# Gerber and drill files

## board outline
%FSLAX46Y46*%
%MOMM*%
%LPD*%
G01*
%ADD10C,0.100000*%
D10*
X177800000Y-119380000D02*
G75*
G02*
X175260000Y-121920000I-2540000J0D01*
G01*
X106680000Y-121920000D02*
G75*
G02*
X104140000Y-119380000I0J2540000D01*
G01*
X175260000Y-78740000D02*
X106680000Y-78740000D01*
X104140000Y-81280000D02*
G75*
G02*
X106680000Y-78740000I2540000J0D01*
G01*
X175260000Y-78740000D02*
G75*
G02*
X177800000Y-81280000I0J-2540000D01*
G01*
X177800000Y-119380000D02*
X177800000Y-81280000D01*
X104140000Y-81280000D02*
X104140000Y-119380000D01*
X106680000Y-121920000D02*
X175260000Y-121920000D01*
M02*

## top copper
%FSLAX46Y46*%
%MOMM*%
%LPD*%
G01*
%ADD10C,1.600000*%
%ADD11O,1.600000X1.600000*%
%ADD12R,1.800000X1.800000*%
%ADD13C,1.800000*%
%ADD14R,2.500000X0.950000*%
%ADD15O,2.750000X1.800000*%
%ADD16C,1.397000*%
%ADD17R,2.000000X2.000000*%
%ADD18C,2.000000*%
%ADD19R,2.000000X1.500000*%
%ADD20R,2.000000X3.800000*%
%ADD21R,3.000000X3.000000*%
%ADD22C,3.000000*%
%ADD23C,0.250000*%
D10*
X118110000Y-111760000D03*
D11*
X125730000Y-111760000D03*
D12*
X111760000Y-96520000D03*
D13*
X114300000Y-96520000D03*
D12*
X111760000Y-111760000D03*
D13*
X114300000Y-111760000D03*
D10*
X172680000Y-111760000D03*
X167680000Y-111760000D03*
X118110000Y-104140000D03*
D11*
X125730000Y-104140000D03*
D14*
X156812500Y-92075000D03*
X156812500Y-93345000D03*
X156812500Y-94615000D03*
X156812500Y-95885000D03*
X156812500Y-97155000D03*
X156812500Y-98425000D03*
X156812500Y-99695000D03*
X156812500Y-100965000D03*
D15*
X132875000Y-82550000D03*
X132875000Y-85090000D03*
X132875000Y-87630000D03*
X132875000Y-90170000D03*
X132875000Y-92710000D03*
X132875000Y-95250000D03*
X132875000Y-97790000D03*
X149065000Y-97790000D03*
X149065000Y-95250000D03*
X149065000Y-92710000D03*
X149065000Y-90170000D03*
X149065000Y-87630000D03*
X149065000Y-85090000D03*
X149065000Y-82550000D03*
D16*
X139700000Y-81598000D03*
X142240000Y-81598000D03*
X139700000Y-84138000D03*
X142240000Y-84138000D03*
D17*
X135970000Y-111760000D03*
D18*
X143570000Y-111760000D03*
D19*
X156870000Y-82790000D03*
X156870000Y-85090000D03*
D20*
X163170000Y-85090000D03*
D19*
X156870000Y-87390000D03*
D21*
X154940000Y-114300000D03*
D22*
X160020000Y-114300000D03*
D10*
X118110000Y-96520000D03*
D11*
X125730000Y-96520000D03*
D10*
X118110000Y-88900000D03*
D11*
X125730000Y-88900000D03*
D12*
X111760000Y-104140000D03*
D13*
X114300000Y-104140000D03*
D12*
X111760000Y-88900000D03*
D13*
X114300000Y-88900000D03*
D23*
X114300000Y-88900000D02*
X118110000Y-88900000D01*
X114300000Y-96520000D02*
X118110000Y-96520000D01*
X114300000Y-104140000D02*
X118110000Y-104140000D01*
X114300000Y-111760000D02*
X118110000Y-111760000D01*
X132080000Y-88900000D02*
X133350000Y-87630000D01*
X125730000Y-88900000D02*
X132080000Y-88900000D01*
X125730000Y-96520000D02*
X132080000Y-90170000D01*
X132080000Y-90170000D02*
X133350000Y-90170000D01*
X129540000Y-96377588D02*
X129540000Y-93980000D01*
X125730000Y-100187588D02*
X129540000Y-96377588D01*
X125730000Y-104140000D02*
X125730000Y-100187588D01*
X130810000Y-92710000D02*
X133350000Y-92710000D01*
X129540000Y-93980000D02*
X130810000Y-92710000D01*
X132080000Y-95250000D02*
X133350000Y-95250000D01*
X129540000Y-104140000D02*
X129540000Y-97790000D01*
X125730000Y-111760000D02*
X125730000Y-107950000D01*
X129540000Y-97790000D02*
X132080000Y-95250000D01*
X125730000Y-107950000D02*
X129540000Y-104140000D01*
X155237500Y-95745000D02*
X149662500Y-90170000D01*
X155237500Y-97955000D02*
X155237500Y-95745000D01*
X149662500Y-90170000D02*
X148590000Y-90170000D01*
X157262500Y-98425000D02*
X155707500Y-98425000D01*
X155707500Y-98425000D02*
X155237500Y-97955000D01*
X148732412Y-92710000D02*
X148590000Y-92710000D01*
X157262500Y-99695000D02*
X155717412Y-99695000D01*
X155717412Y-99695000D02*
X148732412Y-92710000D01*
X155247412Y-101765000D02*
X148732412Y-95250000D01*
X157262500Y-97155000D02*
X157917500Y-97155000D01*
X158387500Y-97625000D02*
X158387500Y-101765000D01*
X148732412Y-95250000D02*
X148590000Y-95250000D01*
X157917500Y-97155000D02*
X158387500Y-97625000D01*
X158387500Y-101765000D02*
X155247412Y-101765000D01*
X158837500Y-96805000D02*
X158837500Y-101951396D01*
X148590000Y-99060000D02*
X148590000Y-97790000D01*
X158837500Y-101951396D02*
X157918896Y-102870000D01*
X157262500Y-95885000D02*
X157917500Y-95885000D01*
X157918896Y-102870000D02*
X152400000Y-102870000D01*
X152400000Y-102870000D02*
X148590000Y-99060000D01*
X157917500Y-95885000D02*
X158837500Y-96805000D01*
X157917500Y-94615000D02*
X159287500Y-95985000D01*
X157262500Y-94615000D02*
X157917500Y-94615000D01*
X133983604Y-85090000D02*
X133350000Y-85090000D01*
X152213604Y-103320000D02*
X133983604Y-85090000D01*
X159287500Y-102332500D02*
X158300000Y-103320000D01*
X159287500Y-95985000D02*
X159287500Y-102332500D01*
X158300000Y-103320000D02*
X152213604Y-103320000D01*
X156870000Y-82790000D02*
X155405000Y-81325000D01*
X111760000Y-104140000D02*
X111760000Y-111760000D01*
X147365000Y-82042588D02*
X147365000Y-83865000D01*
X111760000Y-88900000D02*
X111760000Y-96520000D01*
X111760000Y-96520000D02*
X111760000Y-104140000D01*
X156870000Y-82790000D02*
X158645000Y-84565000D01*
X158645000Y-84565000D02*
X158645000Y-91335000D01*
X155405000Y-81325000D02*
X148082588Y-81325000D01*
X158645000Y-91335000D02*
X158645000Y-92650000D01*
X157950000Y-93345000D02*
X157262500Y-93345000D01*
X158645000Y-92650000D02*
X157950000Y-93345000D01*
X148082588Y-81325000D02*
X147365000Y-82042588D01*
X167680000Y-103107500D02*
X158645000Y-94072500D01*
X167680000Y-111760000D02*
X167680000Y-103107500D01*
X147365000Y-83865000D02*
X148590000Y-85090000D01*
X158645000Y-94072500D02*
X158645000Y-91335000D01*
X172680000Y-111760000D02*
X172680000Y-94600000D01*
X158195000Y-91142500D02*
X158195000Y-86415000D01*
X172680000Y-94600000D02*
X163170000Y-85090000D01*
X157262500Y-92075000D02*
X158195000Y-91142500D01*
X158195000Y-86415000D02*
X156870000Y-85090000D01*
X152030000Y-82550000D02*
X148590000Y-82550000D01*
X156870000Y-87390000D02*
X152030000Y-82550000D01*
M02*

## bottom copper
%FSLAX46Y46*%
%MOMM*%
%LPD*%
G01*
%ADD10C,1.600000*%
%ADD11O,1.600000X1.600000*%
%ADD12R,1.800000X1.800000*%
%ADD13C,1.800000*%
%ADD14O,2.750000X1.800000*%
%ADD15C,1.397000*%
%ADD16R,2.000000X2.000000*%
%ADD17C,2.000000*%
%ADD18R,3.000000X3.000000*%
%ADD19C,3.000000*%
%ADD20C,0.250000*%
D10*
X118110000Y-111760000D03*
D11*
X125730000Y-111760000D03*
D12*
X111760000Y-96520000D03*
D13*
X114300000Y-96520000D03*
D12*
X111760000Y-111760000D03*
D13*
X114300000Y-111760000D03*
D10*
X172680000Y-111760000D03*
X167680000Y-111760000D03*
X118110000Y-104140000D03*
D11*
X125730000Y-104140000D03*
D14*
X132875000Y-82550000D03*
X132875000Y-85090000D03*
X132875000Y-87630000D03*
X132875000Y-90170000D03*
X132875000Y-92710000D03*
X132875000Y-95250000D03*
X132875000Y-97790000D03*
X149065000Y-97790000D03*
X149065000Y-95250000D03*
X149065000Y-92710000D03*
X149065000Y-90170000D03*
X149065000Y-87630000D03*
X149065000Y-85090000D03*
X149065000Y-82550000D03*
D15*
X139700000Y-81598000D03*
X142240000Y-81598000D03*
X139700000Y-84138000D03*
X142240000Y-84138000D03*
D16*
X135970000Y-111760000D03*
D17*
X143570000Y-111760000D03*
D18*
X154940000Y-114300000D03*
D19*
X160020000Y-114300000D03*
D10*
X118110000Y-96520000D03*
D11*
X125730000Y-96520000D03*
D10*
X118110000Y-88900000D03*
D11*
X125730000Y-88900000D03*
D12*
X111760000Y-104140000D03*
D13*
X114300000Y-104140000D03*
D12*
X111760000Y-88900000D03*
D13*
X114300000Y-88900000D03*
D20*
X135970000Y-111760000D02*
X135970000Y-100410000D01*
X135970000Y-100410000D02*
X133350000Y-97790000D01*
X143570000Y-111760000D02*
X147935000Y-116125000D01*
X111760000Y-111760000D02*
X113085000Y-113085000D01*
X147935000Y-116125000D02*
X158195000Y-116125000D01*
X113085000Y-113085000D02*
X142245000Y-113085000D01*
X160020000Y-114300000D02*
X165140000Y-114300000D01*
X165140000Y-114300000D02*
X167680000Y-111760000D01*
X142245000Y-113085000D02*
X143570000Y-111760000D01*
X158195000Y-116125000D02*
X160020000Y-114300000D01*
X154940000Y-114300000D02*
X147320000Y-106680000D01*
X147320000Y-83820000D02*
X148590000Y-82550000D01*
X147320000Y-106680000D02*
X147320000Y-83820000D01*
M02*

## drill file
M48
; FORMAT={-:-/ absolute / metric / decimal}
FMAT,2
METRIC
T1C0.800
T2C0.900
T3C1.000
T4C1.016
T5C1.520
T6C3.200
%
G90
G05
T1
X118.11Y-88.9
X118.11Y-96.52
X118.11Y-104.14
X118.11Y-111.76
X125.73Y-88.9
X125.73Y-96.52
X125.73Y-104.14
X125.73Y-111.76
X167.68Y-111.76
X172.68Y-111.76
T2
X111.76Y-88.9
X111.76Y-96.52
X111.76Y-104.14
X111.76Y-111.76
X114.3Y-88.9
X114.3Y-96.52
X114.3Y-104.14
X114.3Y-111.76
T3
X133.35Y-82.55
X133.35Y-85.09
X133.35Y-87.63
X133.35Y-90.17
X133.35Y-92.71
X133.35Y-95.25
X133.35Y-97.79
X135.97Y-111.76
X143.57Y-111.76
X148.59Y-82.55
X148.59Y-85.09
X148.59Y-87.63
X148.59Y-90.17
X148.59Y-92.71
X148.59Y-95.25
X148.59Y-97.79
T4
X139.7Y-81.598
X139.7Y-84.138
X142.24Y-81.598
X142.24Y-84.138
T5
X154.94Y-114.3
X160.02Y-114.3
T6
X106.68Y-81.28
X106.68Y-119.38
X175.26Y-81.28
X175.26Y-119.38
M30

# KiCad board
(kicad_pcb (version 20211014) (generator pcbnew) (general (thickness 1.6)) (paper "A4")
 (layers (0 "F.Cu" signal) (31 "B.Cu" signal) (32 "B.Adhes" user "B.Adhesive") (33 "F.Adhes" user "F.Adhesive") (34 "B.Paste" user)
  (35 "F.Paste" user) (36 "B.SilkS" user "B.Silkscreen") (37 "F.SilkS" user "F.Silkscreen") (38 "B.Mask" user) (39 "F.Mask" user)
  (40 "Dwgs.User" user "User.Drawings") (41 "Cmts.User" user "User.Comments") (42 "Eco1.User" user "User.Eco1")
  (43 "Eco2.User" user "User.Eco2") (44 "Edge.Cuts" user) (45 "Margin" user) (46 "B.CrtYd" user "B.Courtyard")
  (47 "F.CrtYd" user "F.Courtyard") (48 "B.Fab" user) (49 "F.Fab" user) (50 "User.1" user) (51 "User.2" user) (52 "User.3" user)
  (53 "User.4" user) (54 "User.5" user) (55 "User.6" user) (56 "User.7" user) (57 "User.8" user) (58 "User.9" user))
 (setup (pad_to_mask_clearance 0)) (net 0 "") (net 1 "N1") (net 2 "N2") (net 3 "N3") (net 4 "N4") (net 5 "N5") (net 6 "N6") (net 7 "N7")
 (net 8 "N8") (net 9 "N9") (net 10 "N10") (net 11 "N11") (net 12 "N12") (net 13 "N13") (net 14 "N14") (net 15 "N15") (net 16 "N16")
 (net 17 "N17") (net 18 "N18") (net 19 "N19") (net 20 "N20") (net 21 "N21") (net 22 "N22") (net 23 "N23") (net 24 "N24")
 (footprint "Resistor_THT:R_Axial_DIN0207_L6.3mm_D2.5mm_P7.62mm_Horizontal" (layer "F.Cu") (at 118.11 111.76)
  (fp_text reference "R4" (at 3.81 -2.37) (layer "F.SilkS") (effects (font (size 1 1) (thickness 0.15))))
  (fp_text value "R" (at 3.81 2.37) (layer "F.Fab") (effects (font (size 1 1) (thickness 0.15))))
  (pad "1" thru_hole circle (at 0 0) (size 1.6 1.6) (drill 0.8) (layers *.Cu *.Mask) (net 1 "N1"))
  (pad "2" thru_hole oval (at 7.62 0) (size 1.6 1.6) (drill 0.8) (layers *.Cu *.Mask) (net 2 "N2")))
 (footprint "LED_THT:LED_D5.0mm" (layer "F.Cu") (at 111.76 96.52)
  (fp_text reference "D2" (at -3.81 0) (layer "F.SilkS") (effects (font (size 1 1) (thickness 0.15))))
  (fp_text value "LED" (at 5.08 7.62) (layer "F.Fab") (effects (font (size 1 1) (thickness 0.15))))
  (pad "1" thru_hole rect (at 0 0) (size 1.8 1.8) (drill 0.9) (layers *.Cu *.Mask) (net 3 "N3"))
  (pad "2" thru_hole circle (at 2.54 0) (size 1.8 1.8) (drill 0.9) (layers *.Cu *.Mask) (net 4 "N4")))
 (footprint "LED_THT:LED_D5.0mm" (layer "F.Cu") (at 111.76 111.76)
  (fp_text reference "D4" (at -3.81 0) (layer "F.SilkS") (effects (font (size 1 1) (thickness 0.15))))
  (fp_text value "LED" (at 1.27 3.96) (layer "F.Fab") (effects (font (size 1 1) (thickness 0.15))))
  (pad "1" thru_hole rect (at 0 0) (size 1.8 1.8) (drill 0.9) (layers *.Cu *.Mask) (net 3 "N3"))
  (pad "2" thru_hole circle (at 2.54 0) (size 1.8 1.8) (drill 0.9) (layers *.Cu *.Mask) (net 1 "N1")))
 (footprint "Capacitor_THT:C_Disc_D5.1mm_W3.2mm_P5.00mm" (layer "F.Cu") (at 172.68 111.76 180)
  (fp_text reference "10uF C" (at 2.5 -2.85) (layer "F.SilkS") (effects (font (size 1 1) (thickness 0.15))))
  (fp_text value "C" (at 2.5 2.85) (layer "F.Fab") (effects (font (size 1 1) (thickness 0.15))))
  (pad "1" thru_hole circle (at 0 0 180) (size 1.6 1.6) (drill 0.8) (layers *.Cu *.Mask) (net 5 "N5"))
  (pad "2" thru_hole circle (at 5 0 180) (size 1.6 1.6) (drill 0.8) (layers *.Cu *.Mask) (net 3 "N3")))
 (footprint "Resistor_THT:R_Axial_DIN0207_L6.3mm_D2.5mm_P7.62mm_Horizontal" (layer "F.Cu") (at 118.11 104.14)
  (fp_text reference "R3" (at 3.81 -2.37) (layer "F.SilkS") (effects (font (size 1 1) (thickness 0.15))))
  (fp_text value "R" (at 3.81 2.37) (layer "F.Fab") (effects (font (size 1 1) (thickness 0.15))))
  (pad "1" thru_hole circle (at 0 0) (size 1.6 1.6) (drill 0.8) (layers *.Cu *.Mask) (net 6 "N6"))
  (pad "2" thru_hole oval (at 7.62 0) (size 1.6 1.6) (drill 0.8) (layers *.Cu *.Mask) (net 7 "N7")))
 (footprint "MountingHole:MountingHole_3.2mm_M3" (layer "F.Cu") (at 106.68 119.38)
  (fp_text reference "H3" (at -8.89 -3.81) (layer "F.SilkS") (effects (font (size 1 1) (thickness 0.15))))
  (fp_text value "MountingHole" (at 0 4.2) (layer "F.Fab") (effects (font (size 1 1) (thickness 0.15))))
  (pad "" np_thru_hole circle (at 0 0) (size 3.2 3.2) (drill 3.2) (layers *.Cu *.Mask)))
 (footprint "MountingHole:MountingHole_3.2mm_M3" (layer "F.Cu") (at 106.68 81.28)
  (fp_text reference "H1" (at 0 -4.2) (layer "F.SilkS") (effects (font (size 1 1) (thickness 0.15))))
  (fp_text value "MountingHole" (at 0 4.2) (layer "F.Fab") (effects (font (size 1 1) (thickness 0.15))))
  (pad "" np_thru_hole circle (at 0 0) (size 3.2 3.2) (drill 3.2) (layers *.Cu *.Mask)))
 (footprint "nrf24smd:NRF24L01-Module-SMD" (layer "F.Cu") (at 157.5625 96.52 180)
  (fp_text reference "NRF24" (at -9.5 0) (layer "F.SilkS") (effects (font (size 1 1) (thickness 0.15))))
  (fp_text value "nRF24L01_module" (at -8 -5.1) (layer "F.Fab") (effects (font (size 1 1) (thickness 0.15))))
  (pad "1" smd rect locked (at 0.3 4.445 180) (size 2.5 0.95) (drill (offset 0.45 0)) (layers "F.Cu" "F.Paste" "F.Mask") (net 5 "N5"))
  (pad "2" smd rect locked (at 0.3 3.175 180) (size 2.5 0.95) (drill (offset 0.45 0)) (layers "F.Cu" "F.Paste" "F.Mask") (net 3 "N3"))
  (pad "3" smd rect locked (at 0.3 1.905 180) (size 2.5 0.95) (drill (offset 0.45 0)) (layers "F.Cu" "F.Paste" "F.Mask") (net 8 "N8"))
  (pad "4" smd rect locked (at 0.3 0.635 180) (size 2.5 0.95) (drill (offset 0.45 0)) (layers "F.Cu" "F.Paste" "F.Mask") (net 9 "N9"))
  (pad "5" smd rect locked (at 0.3 -0.635 180) (size 2.5 0.95) (drill (offset 0.45 0)) (layers "F.Cu" "F.Paste" "F.Mask") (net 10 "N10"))
  (pad "6" smd rect locked (at 0.3 -1.905 180) (size 2.5 0.95) (drill (offset 0.45 0)) (layers "F.Cu" "F.Paste" "F.Mask") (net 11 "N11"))
  (pad "7" smd rect locked (at 0.3 -3.175 180) (size 2.5 0.95) (drill (offset 0.45 0)) (layers "F.Cu" "F.Paste" "F.Mask") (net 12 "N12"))
  (pad "8" smd rect locked (at 0.3 -4.445 180) (size 2.5 0.95) (drill (offset 0.45 0)) (layers "F.Cu" "F.Paste" "F.Mask") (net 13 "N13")))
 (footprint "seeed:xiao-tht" (layer "F.Cu") (at 140.97 90.17)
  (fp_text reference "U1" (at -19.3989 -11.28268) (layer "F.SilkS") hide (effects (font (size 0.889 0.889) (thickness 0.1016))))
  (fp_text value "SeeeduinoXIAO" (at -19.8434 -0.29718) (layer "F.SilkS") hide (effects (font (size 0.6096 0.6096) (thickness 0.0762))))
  (pad "1" thru_hole oval (at -7.62 -7.62) (size 2.75 1.8) (drill 1 (offset -0.475 0)) (layers *.Cu *.Mask) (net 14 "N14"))
  (pad "2" thru_hole oval (at -7.62 -5.08) (size 2.75 1.8) (drill 1 (offset -0.475 0)) (layers *.Cu *.Mask) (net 8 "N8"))
  (pad "3" thru_hole oval (at -7.62 -2.54) (size 2.75 1.8) (drill 1 (offset -0.475 0)) (layers *.Cu *.Mask) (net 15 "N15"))
  (pad "4" thru_hole oval (at -7.62 0) (size 2.75 1.8) (drill 1 (offset -0.475 0)) (layers *.Cu *.Mask) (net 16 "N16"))
  (pad "5" thru_hole oval (at -7.62 2.54) (size 2.75 1.8) (drill 1 (offset -0.475 0)) (layers *.Cu *.Mask) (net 7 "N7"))
  (pad "6" thru_hole oval (at -7.62 5.08) (size 2.75 1.8) (drill 1 (offset -0.475 0)) (layers *.Cu *.Mask) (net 2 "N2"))
  (pad "7" thru_hole oval (at -7.62 7.62) (size 2.75 1.8) (drill 1 (offset -0.475 0)) (layers *.Cu *.Mask) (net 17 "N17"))
  (pad "8" thru_hole oval (at 7.62 7.62 180) (size 2.75 1.8) (drill 1 (offset -0.475 0)) (layers *.Cu *.Mask) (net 9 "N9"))
  (pad "9" thru_hole oval (at 7.62 5.08 180) (size 2.75 1.8) (drill 1 (offset -0.475 0)) (layers *.Cu *.Mask) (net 10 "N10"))
  (pad "10" thru_hole oval (at 7.62 2.54 180) (size 2.75 1.8) (drill 1 (offset -0.475 0)) (layers *.Cu *.Mask) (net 12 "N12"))
  (pad "11" thru_hole oval (at 7.62 0 180) (size 2.75 1.8) (drill 1 (offset -0.475 0)) (layers *.Cu *.Mask) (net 11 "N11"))
  (pad "12" thru_hole oval (at 7.62 -2.54 180) (size 2.75 1.8) (drill 1 (offset -0.475 0)) (layers *.Cu *.Mask) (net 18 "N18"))
  (pad "13" thru_hole oval (at 7.62 -5.08 180) (size 2.75 1.8) (drill 1 (offset -0.475 0)) (layers *.Cu *.Mask) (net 3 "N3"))
  (pad "14" thru_hole oval (at 7.62 -7.62 180) (size 2.75 1.8) (drill 1 (offset -0.475 0)) (layers *.Cu *.Mask) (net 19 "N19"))
  (pad "15" thru_hole circle (at -1.27 -8.572 90) (size 1.397 1.397) (drill 1.016) (layers *.Cu *.Mask) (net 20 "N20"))
  (pad "16" thru_hole circle (at 1.27 -8.572 90) (size 1.397 1.397) (drill 1.016) (layers *.Cu *.Mask) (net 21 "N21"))
  (pad "17" thru_hole circle (at -1.27 -6.032 90) (size 1.397 1.397) (drill 1.016) (layers *.Cu *.Mask) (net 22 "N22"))
  (pad "18" thru_hole circle (at 1.27 -6.032 90) (size 1.397 1.397) (drill 1.016) (layers *.Cu *.Mask) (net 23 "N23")))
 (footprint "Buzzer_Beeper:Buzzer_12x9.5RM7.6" (layer "F.Cu") (at 135.97 111.76)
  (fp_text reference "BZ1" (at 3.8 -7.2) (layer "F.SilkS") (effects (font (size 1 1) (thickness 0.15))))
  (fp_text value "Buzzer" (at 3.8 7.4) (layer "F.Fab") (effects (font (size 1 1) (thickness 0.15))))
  (pad "1" thru_hole rect (at 0 0) (size 2 2) (drill 1) (layers *.Cu *.Mask) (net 17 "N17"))
  (pad "2" thru_hole circle (at 7.6 0) (size 2 2) (drill 1) (layers *.Cu *.Mask) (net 3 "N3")))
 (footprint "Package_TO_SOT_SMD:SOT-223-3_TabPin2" (layer "F.Cu") (at 160.02 85.09)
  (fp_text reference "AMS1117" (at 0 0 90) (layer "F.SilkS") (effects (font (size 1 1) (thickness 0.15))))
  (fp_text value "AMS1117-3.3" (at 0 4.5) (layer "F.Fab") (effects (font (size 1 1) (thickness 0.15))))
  (pad "1" smd rect (at -3.15 -2.3) (size 2 1.5) (layers "F.Cu" "F.Paste" "F.Mask") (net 3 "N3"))
  (pad "2" smd rect (at -3.15 0) (size 2 1.5) (layers "F.Cu" "F.Paste" "F.Mask") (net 5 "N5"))
  (pad "2" smd rect (at 3.15 0) (size 2 3.8) (layers "F.Cu" "F.Paste" "F.Mask") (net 5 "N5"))
  (pad "3" smd rect (at -3.15 2.3) (size 2 1.5) (layers "F.Cu" "F.Paste" "F.Mask") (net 19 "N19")))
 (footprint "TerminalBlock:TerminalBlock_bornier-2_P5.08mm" (layer "F.Cu") (at 154.94 114.3)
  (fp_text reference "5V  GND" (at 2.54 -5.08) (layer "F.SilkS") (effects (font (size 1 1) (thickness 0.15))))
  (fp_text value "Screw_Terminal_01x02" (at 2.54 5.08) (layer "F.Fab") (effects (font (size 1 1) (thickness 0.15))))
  (pad "1" thru_hole rect (at 0 0) (size 3 3) (drill 1.52) (layers *.Cu *.Mask) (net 19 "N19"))
  (pad "2" thru_hole circle (at 5.08 0) (size 3 3) (drill 1.52) (layers *.Cu *.Mask) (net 3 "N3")))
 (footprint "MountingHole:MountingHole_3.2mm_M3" (layer "F.Cu") (at 175.26 81.28)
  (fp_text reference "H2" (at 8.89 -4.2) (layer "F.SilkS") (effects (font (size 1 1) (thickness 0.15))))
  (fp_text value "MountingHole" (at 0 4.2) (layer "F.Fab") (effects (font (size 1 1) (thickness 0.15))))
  (pad "" np_thru_hole circle (at 0 0) (size 3.2 3.2) (drill 3.2) (layers *.Cu *.Mask)))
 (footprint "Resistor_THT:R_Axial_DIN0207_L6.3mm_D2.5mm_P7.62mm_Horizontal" (layer "F.Cu") (at 118.11 96.52)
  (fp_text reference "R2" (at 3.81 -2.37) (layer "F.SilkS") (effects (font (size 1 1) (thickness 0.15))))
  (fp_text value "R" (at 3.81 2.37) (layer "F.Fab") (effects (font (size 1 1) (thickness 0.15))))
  (pad "1" thru_hole circle (at 0 0) (size 1.6 1.6) (drill 0.8) (layers *.Cu *.Mask) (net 4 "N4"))
  (pad "2" thru_hole oval (at 7.62 0) (size 1.6 1.6) (drill 0.8) (layers *.Cu *.Mask) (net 16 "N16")))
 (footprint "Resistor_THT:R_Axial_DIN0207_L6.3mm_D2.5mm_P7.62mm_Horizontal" (layer "F.Cu") (at 118.11 88.9)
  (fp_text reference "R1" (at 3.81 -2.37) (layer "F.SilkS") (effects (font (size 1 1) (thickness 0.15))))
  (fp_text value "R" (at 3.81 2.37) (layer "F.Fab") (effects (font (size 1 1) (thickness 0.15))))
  (pad "1" thru_hole circle (at 0 0) (size 1.6 1.6) (drill 0.8) (layers *.Cu *.Mask) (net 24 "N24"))
  (pad "2" thru_hole oval (at 7.62 0) (size 1.6 1.6) (drill 0.8) (layers *.Cu *.Mask) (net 15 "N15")))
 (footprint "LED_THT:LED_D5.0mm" (layer "F.Cu") (at 111.76 104.14)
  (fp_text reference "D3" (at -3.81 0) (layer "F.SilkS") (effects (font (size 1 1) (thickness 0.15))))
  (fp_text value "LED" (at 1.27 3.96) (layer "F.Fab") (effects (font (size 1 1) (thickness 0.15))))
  (pad "1" thru_hole rect (at 0 0) (size 1.8 1.8) (drill 0.9) (layers *.Cu *.Mask) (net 3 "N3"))
  (pad "2" thru_hole circle (at 2.54 0) (size 1.8 1.8) (drill 0.9) (layers *.Cu *.Mask) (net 6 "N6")))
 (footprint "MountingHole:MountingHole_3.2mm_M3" (layer "F.Cu") (at 175.26 119.38)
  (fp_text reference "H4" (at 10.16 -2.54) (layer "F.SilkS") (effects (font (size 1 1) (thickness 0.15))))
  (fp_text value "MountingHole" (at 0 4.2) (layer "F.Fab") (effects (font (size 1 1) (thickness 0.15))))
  (pad "" np_thru_hole circle (at 0 0) (size 3.2 3.2) (drill 3.2) (layers *.Cu *.Mask)))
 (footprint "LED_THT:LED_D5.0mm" (layer "F.Cu") (at 111.76 88.9)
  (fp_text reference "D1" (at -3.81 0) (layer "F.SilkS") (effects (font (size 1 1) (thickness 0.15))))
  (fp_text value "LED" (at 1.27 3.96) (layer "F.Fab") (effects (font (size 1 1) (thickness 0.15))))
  (pad "1" thru_hole rect (at 0 0) (size 1.8 1.8) (drill 0.9) (layers *.Cu *.Mask) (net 3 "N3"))
  (pad "2" thru_hole circle (at 2.54 0) (size 1.8 1.8) (drill 0.9) (layers *.Cu *.Mask) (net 24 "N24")))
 (gr_arc (start 177.8 119.38) (mid 177.056051 121.176051) (end 175.26 121.92) (layer "Edge.Cuts") (width 0.1))
 (gr_arc (start 106.68 121.92) (mid 104.883949 121.176051) (end 104.14 119.38) (layer "Edge.Cuts") (width 0.1))
 (gr_line (start 175.26 78.74) (end 106.68 78.74) (layer "Edge.Cuts") (width 0.1))
 (gr_arc (start 104.14 81.28) (mid 104.883949 79.483949) (end 106.68 78.74) (layer "Edge.Cuts") (width 0.1))
 (gr_arc (start 175.26 78.74) (mid 177.056051 79.483949) (end 177.8 81.28) (layer "Edge.Cuts") (width 0.1))
 (gr_line (start 177.8 119.38) (end 177.8 81.28) (layer "Edge.Cuts") (width 0.1))
 (gr_line (start 104.14 81.28) (end 104.14 119.38) (layer "Edge.Cuts") (width 0.1))
 (gr_line (start 106.68 121.92) (end 175.26 121.92) (layer "Edge.Cuts") (width 0.1))
 (segment (start 114.3 88.9) (end 118.11 88.9) (width 0.25) (layer "F.Cu") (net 24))
 (segment (start 114.3 96.52) (end 118.11 96.52) (width 0.25) (layer "F.Cu") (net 4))
 (segment (start 114.3 104.14) (end 118.11 104.14) (width 0.25) (layer "F.Cu") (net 6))
 (segment (start 114.3 111.76) (end 118.11 111.76) (width 0.25) (layer "F.Cu") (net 1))
 (segment (start 132.08 88.9) (end 133.35 87.63) (width 0.25) (layer "F.Cu") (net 15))
 (segment (start 125.73 88.9) (end 132.08 88.9) (width 0.25) (layer "F.Cu") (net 15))
 (segment (start 125.73 96.52) (end 132.08 90.17) (width 0.25) (layer "F.Cu") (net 16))
 (segment (start 132.08 90.17) (end 133.35 90.17) (width 0.25) (layer "F.Cu") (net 16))
 (segment (start 129.54 96.377588) (end 129.54 93.98) (width 0.25) (layer "F.Cu") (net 7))
 (segment (start 125.73 100.187588) (end 129.54 96.377588) (width 0.25) (layer "F.Cu") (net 7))
 (segment (start 125.73 104.14) (end 125.73 100.187588) (width 0.25) (layer "F.Cu") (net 7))
 (segment (start 130.81 92.71) (end 133.35 92.71) (width 0.25) (layer "F.Cu") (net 7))
 (segment (start 129.54 93.98) (end 130.81 92.71) (width 0.25) (layer "F.Cu") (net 7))
 (segment (start 132.08 95.25) (end 133.35 95.25) (width 0.25) (layer "F.Cu") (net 2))
 (segment (start 129.54 104.14) (end 129.54 97.79) (width 0.25) (layer "F.Cu") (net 2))
 (segment (start 125.73 111.76) (end 125.73 107.95) (width 0.25) (layer "F.Cu") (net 2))
 (segment (start 129.54 97.79) (end 132.08 95.25) (width 0.25) (layer "F.Cu") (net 2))
 (segment (start 125.73 107.95) (end 129.54 104.14) (width 0.25) (layer "F.Cu") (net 2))
 (segment (start 155.2375 95.745) (end 149.6625 90.17) (width 0.25) (layer "F.Cu") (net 11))
 (segment (start 155.2375 97.955) (end 155.2375 95.745) (width 0.25) (layer "F.Cu") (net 11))
 (segment (start 149.6625 90.17) (end 148.59 90.17) (width 0.25) (layer "F.Cu") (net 11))
 (segment (start 157.2625 98.425) (end 155.7075 98.425) (width 0.25) (layer "F.Cu") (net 11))
 (segment (start 155.7075 98.425) (end 155.2375 97.955) (width 0.25) (layer "F.Cu") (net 11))
 (segment (start 148.732412 92.71) (end 148.59 92.71) (width 0.25) (layer "F.Cu") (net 12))
 (segment (start 157.2625 99.695) (end 155.717412 99.695) (width 0.25) (layer "F.Cu") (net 12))
 (segment (start 155.717412 99.695) (end 148.732412 92.71) (width 0.25) (layer "F.Cu") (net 12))
 (segment (start 155.247412 101.765) (end 148.732412 95.25) (width 0.25) (layer "F.Cu") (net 10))
 (segment (start 157.2625 97.155) (end 157.9175 97.155) (width 0.25) (layer "F.Cu") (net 10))
 (segment (start 158.3875 97.625) (end 158.3875 101.765) (width 0.25) (layer "F.Cu") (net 10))
 (segment (start 148.732412 95.25) (end 148.59 95.25) (width 0.25) (layer "F.Cu") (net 10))
 (segment (start 157.9175 97.155) (end 158.3875 97.625) (width 0.25) (layer "F.Cu") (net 10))
 (segment (start 158.3875 101.765) (end 155.247412 101.765) (width 0.25) (layer "F.Cu") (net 10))
 (segment (start 158.8375 96.805) (end 158.8375 101.951396) (width 0.25) (layer "F.Cu") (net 9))
 (segment (start 148.59 99.06) (end 148.59 97.79) (width 0.25) (layer "F.Cu") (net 9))
 (segment (start 158.8375 101.951396) (end 157.918896 102.87) (width 0.25) (layer "F.Cu") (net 9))
 (segment (start 157.2625 95.885) (end 157.9175 95.885) (width 0.25) (layer "F.Cu") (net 9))
 (segment (start 157.918896 102.87) (end 152.4 102.87) (width 0.25) (layer "F.Cu") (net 9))
 (segment (start 152.4 102.87) (end 148.59 99.06) (width 0.25) (layer "F.Cu") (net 9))
 (segment (start 157.9175 95.885) (end 158.8375 96.805) (width 0.25) (layer "F.Cu") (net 9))
 (segment (start 157.9175 94.615) (end 159.2875 95.985) (width 0.25) (layer "F.Cu") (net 8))
 (segment (start 157.2625 94.615) (end 157.9175 94.615) (width 0.25) (layer "F.Cu") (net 8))
 (segment (start 133.983604 85.09) (end 133.35 85.09) (width 0.25) (layer "F.Cu") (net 8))
 (segment (start 152.213604 103.32) (end 133.983604 85.09) (width 0.25) (layer "F.Cu") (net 8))
 (segment (start 159.2875 102.3325) (end 158.3 103.32) (width 0.25) (layer "F.Cu") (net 8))
 (segment (start 159.2875 95.985) (end 159.2875 102.3325) (width 0.25) (layer "F.Cu") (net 8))
 (segment (start 158.3 103.32) (end 152.213604 103.32) (width 0.25) (layer "F.Cu") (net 8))
 (segment (start 135.97 111.76) (end 135.97 100.41) (width 0.25) (layer "B.Cu") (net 17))
 (segment (start 135.97 100.41) (end 133.35 97.79) (width 0.25) (layer "B.Cu") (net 17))
 (segment (start 156.87 82.79) (end 155.405 81.325) (width 0.25) (layer "F.Cu") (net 3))
 (segment (start 111.76 104.14) (end 111.76 111.76) (width 0.25) (layer "F.Cu") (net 3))
 (segment (start 147.365 82.042588) (end 147.365 83.865) (width 0.25) (layer "F.Cu") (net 3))
 (segment (start 111.76 88.9) (end 111.76 96.52) (width 0.25) (layer "F.Cu") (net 3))
 (segment (start 111.76 96.52) (end 111.76 104.14) (width 0.25) (layer "F.Cu") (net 3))
 (segment (start 156.87 82.79) (end 158.645 84.565) (width 0.25) (layer "F.Cu") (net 3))
 (segment (start 158.645 84.565) (end 158.645 91.335) (width 0.25) (layer "F.Cu") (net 3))
 (segment (start 155.405 81.325) (end 148.082588 81.325) (width 0.25) (layer "F.Cu") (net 3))
 (segment (start 158.645 91.335) (end 158.645 92.65) (width 0.25) (layer "F.Cu") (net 3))
 (segment (start 157.95 93.345) (end 157.2625 93.345) (width 0.25) (layer "F.Cu") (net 3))
 (segment (start 158.645 92.65) (end 157.95 93.345) (width 0.25) (layer "F.Cu") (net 3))
 (segment (start 148.082588 81.325) (end 147.365 82.042588) (width 0.25) (layer "F.Cu") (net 3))
 (segment (start 167.68 103.1075) (end 158.645 94.0725) (width 0.25) (layer "F.Cu") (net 3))
 (segment (start 167.68 111.76) (end 167.68 103.1075) (width 0.25) (layer "F.Cu") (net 3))
 (segment (start 147.365 83.865) (end 148.59 85.09) (width 0.25) (layer "F.Cu") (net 3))
 (segment (start 158.645 94.0725) (end 158.645 91.335) (width 0.25) (layer "F.Cu") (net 3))
 (segment (start 143.57 111.76) (end 147.935 116.125) (width 0.25) (layer "B.Cu") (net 3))
 (segment (start 111.76 111.76) (end 113.085 113.085) (width 0.25) (layer "B.Cu") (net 3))
 (segment (start 147.935 116.125) (end 158.195 116.125) (width 0.25) (layer "B.Cu") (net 3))
 (segment (start 113.085 113.085) (end 142.245 113.085) (width 0.25) (layer "B.Cu") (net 3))
 (segment (start 160.02 114.3) (end 165.14 114.3) (width 0.25) (layer "B.Cu") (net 3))
 (segment (start 165.14 114.3) (end 167.68 111.76) (width 0.25) (layer "B.Cu") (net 3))
 (segment (start 142.245 113.085) (end 143.57 111.76) (width 0.25) (layer "B.Cu") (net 3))
 (segment (start 158.195 116.125) (end 160.02 114.3) (width 0.25) (layer "B.Cu") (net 3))
 (segment (start 172.68 111.76) (end 172.68 94.6) (width 0.25) (layer "F.Cu") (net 5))
 (segment (start 158.195 91.1425) (end 158.195 86.415) (width 0.25) (layer "F.Cu") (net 5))
 (segment (start 172.68 94.6) (end 163.17 85.09) (width 0.25) (layer "F.Cu") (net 5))
 (segment (start 157.2625 92.075) (end 158.195 91.1425) (width 0.25) (layer "F.Cu") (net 5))
 (segment (start 158.195 86.415) (end 156.87 85.09) (width 0.25) (layer "F.Cu") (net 5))
 (segment (start 152.03 82.55) (end 148.59 82.55) (width 0.25) (layer "F.Cu") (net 19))
 (segment (start 156.87 87.39) (end 152.03 82.55) (width 0.25) (layer "F.Cu") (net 19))
 (segment (start 154.94 114.3) (end 147.32 106.68) (width 0.25) (layer "B.Cu") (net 19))
 (segment (start 147.32 83.82) (end 148.59 82.55) (width 0.25) (layer "B.Cu") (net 19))
 (segment (start 147.32 106.68) (end 147.32 83.82) (width 0.25) (layer "B.Cu") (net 19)))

